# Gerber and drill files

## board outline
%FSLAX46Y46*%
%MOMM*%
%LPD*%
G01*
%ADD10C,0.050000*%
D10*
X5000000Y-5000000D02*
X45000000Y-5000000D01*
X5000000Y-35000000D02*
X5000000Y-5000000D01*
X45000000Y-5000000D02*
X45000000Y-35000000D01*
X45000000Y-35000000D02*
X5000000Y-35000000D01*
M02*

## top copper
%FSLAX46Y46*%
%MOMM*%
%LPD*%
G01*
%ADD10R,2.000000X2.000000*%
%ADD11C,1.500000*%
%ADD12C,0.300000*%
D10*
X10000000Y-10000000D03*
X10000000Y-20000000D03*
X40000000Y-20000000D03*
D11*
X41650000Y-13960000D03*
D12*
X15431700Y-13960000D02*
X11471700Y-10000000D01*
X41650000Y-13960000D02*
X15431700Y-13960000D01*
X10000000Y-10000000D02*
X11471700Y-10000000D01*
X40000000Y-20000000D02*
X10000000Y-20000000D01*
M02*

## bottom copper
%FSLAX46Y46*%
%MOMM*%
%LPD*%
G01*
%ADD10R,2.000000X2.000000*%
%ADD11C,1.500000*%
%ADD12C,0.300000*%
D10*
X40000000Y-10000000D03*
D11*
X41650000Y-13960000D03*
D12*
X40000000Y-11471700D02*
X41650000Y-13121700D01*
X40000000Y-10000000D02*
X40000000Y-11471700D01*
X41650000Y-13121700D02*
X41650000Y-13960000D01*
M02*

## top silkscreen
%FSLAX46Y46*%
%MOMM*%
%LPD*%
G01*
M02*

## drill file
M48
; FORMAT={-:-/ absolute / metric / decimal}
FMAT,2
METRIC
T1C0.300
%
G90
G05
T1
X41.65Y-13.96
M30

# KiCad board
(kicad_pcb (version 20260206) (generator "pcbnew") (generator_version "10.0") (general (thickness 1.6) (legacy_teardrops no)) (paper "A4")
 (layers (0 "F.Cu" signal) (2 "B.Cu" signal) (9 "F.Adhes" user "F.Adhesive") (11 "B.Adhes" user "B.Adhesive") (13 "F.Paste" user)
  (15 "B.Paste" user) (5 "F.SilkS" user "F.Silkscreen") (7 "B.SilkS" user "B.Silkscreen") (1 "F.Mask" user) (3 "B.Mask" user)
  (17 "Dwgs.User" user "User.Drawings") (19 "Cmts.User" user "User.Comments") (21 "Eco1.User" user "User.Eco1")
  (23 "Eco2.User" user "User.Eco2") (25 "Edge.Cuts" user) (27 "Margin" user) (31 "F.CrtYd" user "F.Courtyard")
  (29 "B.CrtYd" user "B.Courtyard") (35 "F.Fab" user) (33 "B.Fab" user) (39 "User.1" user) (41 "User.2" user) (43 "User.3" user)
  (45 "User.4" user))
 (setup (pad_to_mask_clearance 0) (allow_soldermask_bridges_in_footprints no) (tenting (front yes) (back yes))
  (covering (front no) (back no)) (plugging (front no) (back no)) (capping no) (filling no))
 (gr_line (start 5 5) (end 45 5) (stroke (width 0.05) (type default)) (layer "Edge.Cuts"))
 (gr_line (start 5 35) (end 5 5) (stroke (width 0.05) (type default)) (layer "Edge.Cuts"))
 (gr_line (start 45 5) (end 45 35) (stroke (width 0.05) (type default)) (layer "Edge.Cuts"))
 (gr_line (start 45 35) (end 5 35) (stroke (width 0.05) (type default)) (layer "Edge.Cuts"))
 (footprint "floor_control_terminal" (layer "F.Cu") (at 10 10)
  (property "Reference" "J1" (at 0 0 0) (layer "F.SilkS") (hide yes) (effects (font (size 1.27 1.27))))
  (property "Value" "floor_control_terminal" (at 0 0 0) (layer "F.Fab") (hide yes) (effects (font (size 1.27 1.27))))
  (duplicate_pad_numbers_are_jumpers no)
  (pad "1" smd rect (at 0 0) (size 2 2) (layers "F.Cu" "F.Paste" "F.Mask") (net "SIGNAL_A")))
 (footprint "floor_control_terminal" (layer "B.Cu") (at 40 10)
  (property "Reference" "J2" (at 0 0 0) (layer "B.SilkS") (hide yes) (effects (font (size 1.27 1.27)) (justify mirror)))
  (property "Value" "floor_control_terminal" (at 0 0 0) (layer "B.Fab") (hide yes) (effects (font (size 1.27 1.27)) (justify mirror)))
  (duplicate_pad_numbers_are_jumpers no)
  (pad "1" smd rect (at 0 0) (size 2 2) (layers "B.Cu" "B.Paste" "B.Mask") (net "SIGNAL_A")))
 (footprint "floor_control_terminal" (layer "F.Cu") (at 10 20)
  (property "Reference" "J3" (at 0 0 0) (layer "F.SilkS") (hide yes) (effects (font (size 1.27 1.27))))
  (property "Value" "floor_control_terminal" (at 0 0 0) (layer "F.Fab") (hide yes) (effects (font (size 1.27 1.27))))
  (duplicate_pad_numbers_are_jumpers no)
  (pad "1" smd rect (at 0 0) (size 2 2) (layers "F.Cu" "F.Paste" "F.Mask") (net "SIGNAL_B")))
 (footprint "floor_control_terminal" (layer "F.Cu") (at 40 20)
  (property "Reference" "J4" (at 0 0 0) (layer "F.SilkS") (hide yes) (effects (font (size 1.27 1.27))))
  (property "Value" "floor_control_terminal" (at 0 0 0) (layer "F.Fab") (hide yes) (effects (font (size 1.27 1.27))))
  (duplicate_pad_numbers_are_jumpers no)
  (pad "1" smd rect (at 0 0) (size 2 2) (layers "F.Cu" "F.Paste" "F.Mask") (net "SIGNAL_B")))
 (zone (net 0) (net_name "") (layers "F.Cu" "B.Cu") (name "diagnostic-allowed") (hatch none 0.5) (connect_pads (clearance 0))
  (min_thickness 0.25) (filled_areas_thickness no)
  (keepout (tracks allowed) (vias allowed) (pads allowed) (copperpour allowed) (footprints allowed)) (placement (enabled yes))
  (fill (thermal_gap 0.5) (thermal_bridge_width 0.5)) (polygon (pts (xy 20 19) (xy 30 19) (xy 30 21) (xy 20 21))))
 (segment (start 15.4317 13.96) (end 11.4717 10) (width 0.3) (layer "F.Cu") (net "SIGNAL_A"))
 (segment (start 41.65 13.96) (end 15.4317 13.96) (width 0.3) (layer "F.Cu") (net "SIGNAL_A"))
 (segment (start 10 10) (end 11.4717 10) (width 0.3) (layer "F.Cu") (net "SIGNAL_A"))
 (via (at 41.65 13.96) (size 1.5) (drill 0.3) (layers "F.Cu" "B.Cu") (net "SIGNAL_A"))
 (segment (start 40 11.4717) (end 41.65 13.1217) (width 0.3) (layer "B.Cu") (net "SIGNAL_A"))
 (segment (start 40 10) (end 40 11.4717) (width 0.3) (layer "B.Cu") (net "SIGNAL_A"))
 (segment (start 41.65 13.1217) (end 41.65 13.96) (width 0.3) (layer "B.Cu") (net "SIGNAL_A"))
 (segment (start 40 20) (end 10 20) (width 0.3) (layer "F.Cu") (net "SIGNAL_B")))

